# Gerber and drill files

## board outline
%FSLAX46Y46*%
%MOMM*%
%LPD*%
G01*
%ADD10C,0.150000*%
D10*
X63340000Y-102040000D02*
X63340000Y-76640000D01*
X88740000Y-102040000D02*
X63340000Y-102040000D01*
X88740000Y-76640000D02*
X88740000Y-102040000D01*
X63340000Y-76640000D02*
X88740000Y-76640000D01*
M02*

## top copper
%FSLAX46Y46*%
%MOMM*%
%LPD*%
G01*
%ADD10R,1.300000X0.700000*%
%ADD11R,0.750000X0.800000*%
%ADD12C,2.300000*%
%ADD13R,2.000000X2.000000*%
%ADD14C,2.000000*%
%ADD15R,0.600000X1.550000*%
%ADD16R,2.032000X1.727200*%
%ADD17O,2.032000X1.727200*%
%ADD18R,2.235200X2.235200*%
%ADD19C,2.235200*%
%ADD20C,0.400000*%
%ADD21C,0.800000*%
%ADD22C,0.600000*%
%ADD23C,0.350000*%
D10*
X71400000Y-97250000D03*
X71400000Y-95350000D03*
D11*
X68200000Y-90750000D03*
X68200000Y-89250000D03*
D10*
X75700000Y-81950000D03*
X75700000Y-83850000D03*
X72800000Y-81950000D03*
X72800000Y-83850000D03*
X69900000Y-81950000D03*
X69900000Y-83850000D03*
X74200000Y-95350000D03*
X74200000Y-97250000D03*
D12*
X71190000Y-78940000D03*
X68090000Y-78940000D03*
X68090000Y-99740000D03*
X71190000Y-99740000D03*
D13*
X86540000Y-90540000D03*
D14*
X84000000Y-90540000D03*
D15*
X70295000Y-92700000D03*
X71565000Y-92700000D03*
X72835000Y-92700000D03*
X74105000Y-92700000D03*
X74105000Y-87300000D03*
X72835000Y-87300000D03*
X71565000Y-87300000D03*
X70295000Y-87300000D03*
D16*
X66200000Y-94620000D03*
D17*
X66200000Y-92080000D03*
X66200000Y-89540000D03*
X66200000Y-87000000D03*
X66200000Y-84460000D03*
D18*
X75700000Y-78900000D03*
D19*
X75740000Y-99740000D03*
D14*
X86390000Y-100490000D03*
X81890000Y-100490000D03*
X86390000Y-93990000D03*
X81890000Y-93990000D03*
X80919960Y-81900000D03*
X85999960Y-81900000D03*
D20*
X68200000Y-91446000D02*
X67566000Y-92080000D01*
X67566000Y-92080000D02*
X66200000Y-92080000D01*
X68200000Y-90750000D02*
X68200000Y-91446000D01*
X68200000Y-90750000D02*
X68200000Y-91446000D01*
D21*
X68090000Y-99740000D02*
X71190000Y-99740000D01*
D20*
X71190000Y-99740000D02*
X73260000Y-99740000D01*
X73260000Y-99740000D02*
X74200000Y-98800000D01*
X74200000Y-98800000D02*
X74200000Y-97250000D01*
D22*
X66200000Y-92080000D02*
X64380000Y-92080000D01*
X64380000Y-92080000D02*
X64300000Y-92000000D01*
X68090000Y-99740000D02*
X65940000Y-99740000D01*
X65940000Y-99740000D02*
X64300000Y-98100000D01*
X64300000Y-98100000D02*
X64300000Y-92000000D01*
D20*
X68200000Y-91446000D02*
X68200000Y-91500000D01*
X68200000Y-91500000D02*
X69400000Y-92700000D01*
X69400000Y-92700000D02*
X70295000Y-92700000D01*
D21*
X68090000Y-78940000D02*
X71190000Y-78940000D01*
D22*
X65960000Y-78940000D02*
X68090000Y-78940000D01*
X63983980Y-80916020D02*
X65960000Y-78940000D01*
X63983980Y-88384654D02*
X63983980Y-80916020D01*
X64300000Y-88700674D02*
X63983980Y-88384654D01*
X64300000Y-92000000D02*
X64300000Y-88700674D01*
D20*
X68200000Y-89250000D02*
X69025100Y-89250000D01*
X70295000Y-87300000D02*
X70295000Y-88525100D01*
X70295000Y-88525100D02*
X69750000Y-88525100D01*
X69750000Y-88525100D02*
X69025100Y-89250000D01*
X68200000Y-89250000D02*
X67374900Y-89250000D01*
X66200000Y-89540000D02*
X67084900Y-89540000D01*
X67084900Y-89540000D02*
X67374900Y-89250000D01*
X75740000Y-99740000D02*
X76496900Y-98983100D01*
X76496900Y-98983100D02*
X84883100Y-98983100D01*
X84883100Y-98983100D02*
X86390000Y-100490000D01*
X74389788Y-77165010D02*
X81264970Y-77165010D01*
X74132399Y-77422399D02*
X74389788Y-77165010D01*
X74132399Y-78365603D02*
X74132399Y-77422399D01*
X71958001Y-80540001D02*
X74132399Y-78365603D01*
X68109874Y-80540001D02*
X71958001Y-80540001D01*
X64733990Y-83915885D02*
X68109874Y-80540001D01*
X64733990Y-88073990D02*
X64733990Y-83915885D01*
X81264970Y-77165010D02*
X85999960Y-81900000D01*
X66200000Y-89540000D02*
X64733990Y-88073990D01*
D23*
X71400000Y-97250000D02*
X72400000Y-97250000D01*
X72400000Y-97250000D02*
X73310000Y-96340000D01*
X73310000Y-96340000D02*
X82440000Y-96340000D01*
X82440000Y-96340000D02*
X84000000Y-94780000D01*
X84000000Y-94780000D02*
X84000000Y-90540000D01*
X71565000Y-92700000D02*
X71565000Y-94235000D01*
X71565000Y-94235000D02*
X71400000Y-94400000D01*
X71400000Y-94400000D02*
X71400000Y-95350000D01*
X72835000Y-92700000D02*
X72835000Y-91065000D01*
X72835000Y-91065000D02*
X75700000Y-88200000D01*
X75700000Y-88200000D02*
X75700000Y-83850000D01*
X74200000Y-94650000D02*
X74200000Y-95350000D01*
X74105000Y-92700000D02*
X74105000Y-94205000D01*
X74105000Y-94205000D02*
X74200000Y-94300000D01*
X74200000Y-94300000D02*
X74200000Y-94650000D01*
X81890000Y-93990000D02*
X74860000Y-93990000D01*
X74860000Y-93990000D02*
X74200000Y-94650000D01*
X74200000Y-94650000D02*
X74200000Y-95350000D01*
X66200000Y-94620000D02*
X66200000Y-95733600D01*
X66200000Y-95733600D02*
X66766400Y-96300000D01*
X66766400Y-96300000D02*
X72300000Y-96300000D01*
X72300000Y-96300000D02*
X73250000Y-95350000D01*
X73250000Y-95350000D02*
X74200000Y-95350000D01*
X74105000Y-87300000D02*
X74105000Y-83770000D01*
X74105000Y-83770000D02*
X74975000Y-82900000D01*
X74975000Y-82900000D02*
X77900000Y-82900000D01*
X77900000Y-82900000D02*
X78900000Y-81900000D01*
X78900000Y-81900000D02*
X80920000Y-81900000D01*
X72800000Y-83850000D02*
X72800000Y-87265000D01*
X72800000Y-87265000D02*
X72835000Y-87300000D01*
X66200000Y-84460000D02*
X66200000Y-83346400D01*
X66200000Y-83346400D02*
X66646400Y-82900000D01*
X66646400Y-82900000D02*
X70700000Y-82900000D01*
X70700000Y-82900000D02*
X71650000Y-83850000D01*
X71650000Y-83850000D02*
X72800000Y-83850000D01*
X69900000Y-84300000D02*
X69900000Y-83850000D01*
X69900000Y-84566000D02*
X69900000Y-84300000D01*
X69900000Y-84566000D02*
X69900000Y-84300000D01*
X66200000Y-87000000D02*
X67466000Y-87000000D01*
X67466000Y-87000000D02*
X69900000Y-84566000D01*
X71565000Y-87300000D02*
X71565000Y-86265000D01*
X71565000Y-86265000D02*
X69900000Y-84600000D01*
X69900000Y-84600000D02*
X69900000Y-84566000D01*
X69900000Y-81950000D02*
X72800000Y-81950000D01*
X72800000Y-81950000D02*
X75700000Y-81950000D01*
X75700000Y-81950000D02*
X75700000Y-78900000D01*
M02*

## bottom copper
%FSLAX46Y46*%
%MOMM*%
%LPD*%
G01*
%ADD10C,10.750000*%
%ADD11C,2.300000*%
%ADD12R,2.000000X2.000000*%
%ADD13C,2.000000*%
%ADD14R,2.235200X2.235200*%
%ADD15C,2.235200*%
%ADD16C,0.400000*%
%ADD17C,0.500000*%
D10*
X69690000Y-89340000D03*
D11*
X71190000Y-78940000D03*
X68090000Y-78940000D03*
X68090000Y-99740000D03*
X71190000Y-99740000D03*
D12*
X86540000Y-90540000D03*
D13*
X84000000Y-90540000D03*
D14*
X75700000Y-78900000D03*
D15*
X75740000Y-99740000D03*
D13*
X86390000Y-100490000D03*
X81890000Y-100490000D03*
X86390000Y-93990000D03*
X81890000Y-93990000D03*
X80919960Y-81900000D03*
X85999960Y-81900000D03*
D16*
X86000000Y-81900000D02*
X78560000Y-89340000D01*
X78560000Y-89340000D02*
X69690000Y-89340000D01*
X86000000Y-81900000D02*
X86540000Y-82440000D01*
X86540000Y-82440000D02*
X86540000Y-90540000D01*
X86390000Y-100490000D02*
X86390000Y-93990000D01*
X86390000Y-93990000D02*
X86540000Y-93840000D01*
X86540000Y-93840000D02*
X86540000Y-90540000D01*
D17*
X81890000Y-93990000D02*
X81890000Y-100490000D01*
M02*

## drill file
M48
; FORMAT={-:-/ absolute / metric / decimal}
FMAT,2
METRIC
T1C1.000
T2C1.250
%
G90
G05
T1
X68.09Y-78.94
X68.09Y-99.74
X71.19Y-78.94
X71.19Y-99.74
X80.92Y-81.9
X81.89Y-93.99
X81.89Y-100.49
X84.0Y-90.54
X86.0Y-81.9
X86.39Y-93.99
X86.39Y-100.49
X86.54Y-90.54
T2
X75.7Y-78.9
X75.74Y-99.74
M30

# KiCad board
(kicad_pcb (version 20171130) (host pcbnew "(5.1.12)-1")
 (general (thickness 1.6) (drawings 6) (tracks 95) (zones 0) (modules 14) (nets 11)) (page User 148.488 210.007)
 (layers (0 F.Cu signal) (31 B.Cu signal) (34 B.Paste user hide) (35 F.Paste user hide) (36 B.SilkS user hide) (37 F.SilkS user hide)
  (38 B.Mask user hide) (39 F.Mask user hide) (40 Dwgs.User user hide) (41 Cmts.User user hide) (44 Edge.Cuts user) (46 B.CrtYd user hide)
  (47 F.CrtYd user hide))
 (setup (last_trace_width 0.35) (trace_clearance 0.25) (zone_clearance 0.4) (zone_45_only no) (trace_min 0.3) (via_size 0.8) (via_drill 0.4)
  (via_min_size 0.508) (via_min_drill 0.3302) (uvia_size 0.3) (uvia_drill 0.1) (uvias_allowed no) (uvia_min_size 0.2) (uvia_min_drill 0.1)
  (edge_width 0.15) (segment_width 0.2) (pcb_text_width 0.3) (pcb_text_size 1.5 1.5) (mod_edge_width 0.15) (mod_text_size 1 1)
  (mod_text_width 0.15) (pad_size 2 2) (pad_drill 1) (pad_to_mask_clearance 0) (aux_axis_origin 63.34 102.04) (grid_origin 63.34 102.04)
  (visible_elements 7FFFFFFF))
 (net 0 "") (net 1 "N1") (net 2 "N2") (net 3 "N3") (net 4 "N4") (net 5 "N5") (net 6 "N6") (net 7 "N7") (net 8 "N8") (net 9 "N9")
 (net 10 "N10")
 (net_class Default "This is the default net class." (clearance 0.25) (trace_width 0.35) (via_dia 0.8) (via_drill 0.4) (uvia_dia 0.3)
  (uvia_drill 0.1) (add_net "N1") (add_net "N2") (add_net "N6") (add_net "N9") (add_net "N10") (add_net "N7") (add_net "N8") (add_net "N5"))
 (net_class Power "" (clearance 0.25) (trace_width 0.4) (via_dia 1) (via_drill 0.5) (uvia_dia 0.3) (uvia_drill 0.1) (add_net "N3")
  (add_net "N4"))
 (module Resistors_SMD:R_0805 (layer F.Cu) (at 71.4 96.3 90)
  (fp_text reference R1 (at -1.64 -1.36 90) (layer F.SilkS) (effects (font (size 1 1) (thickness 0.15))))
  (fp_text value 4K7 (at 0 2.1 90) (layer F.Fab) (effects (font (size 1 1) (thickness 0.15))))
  (pad 1 smd rect (at -0.95 0 90) (size 0.7 1.3) (layers F.Cu F.Paste F.Mask) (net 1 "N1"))
  (pad 2 smd rect (at 0.95 0 90) (size 0.7 1.3) (layers F.Cu F.Paste F.Mask) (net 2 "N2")))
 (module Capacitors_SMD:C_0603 (layer F.Cu) (at 68.2 90 90)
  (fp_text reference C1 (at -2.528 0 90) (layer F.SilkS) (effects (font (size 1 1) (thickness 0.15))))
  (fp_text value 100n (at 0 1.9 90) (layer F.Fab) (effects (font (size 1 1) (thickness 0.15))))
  (pad 1 smd rect (at -0.75 0 90) (size 0.8 0.75) (layers F.Cu F.Paste F.Mask) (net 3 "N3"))
  (pad 2 smd rect (at 0.75 0 90) (size 0.8 0.75) (layers F.Cu F.Paste F.Mask) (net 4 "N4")))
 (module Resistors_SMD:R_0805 (layer F.Cu) (at 75.7 82.9 270)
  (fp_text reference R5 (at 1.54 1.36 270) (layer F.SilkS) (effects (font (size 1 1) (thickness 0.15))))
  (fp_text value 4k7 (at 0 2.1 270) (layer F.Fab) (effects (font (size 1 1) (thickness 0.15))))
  (pad 1 smd rect (at -0.95 0 270) (size 0.7 1.3) (layers F.Cu F.Paste F.Mask) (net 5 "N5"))
  (pad 2 smd rect (at 0.95 0 270) (size 0.7 1.3) (layers F.Cu F.Paste F.Mask) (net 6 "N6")))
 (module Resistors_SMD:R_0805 (layer F.Cu) (at 72.8 82.9 270)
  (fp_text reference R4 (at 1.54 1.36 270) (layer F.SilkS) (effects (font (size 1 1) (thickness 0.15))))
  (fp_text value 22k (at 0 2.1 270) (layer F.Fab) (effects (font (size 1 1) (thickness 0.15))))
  (pad 1 smd rect (at -0.95 0 270) (size 0.7 1.3) (layers F.Cu F.Paste F.Mask) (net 5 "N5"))
  (pad 2 smd rect (at 0.95 0 270) (size 0.7 1.3) (layers F.Cu F.Paste F.Mask) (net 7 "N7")))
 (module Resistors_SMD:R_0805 (layer F.Cu) (at 69.9 82.9 270)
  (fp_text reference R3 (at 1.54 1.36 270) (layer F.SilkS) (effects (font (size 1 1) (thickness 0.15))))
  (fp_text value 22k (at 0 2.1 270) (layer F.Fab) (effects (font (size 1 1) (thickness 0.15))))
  (pad 1 smd rect (at -0.95 0 270) (size 0.7 1.3) (layers F.Cu F.Paste F.Mask) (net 5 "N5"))
  (pad 2 smd rect (at 0.95 0 270) (size 0.7 1.3) (layers F.Cu F.Paste F.Mask) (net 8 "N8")))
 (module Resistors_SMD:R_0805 (layer F.Cu) (at 74.2 96.3 270)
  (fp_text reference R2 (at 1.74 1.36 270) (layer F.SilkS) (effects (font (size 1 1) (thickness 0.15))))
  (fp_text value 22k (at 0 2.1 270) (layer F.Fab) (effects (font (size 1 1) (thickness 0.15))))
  (pad 1 smd rect (at -0.95 0 270) (size 0.7 1.3) (layers F.Cu F.Paste F.Mask) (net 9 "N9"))
  (pad 2 smd rect (at 0.95 0 270) (size 0.7 1.3) (layers F.Cu F.Paste F.Mask) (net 3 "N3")))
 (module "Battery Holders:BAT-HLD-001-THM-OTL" (layer B.Cu) (at 69.69 89.34 90)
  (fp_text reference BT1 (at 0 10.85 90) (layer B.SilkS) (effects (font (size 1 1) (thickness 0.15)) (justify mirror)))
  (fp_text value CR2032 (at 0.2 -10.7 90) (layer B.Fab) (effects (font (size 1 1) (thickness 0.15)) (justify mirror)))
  (pad 2 smd circle (at 0 0 90) (size 10.75 10.75) (layers B.Cu B.Mask) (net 4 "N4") (solder_mask_margin 4) (clearance 2.5) (zone_connect 1)
   (thermal_gap 4))
  (pad 1 thru_hole circle (at 10.4 1.5 90) (size 2.3 2.3) (drill 1) (layers *.Cu *.Mask B.SilkS) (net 3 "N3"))
  (pad 1 thru_hole circle (at 10.4 -1.6 90) (size 2.3 2.3) (drill 1) (layers *.Cu *.Mask B.SilkS) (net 3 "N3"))
  (pad 1 thru_hole circle (at -10.4 -1.6 90) (size 2.3 2.3) (drill 1) (layers *.Cu *.Mask B.SilkS) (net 3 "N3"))
  (pad 1 thru_hole circle (at -10.4 1.5 90) (size 2.3 2.3) (drill 1) (layers *.Cu *.Mask B.SilkS) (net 3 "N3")))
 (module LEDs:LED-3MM (layer F.Cu) (at 86.54 90.54 180)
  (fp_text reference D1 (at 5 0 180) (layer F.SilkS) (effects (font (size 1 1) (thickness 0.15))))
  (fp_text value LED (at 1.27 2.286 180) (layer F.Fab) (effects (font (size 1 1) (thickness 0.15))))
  (pad 1 thru_hole rect (at 0 0 270) (size 2 2) (drill 1) (layers *.Cu *.Mask F.SilkS) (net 4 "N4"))
  (pad 2 thru_hole circle (at 2.54 0 180) (size 2 2) (drill 1) (layers *.Cu *.Mask F.SilkS) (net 1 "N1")))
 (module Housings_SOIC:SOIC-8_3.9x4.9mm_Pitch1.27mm (layer F.Cu) (at 72.2 90 90)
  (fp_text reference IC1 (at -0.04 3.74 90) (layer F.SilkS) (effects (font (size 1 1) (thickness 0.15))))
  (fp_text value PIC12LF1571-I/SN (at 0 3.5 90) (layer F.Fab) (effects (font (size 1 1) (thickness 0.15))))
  (pad 1 smd rect (at -2.7 -1.905 90) (size 1.55 0.6) (layers F.Cu F.Paste F.Mask) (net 3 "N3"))
  (pad 2 smd rect (at -2.7 -0.635 90) (size 1.55 0.6) (layers F.Cu F.Paste F.Mask) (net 2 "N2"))
  (pad 3 smd rect (at -2.7 0.635 90) (size 1.55 0.6) (layers F.Cu F.Paste F.Mask) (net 6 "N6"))
  (pad 4 smd rect (at -2.7 1.905 90) (size 1.55 0.6) (layers F.Cu F.Paste F.Mask) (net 9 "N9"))
  (pad 5 smd rect (at 2.7 1.905 90) (size 1.55 0.6) (layers F.Cu F.Paste F.Mask) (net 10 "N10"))
  (pad 6 smd rect (at 2.7 0.635 90) (size 1.55 0.6) (layers F.Cu F.Paste F.Mask) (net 7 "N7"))
  (pad 7 smd rect (at 2.7 -0.635 90) (size 1.55 0.6) (layers F.Cu F.Paste F.Mask) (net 8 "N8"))
  (pad 8 smd rect (at 2.7 -1.905 90) (size 1.55 0.6) (layers F.Cu F.Paste F.Mask) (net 4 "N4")))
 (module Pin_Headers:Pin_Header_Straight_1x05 (layer F.Cu) (at 66.2 94.62 180)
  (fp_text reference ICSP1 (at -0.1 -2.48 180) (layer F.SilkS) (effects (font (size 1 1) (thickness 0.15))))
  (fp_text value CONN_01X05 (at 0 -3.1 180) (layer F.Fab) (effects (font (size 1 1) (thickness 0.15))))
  (pad 1 smd rect (at 0 0 180) (size 2.032 1.7272) (layers F.Cu F.Mask) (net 9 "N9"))
  (pad 2 smd oval (at 0 2.54 180) (size 2.032 1.7272) (layers F.Cu F.Mask) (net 3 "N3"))
  (pad 3 smd oval (at 0 5.08 180) (size 2.032 1.7272) (layers F.Cu F.Mask) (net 4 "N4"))
  (pad 4 smd oval (at 0 7.62 180) (size 2.032 1.7272) (layers F.Cu F.Mask) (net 8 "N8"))
  (pad 5 smd oval (at 0 10.16 180) (size 2.032 1.7272) (layers F.Cu F.Mask) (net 7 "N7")))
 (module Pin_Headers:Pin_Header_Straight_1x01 (layer F.Cu) (at 75.7 78.9)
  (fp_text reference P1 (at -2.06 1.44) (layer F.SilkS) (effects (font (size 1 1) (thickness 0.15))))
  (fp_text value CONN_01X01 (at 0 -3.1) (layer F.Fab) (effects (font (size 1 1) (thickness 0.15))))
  (pad 1 thru_hole rect (at 0 0) (size 2.2352 2.2352) (drill 1.25) (layers *.Cu *.Mask F.SilkS) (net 5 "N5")))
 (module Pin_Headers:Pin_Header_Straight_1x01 (layer F.Cu) (at 75.74 99.74)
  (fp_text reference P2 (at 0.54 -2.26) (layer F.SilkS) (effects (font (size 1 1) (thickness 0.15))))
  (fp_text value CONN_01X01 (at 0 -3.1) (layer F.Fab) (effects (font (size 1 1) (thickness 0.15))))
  (pad 1 thru_hole circle (at 0 0) (size 2.2352 2.2352) (drill 1.25) (layers *.Cu *.Mask F.SilkS) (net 4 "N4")))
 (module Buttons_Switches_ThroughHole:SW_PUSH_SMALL (layer F.Cu) (at 84.14 97.24 270)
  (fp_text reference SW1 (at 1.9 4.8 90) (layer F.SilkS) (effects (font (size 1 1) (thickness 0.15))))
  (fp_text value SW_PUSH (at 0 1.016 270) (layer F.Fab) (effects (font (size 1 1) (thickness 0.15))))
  (pad 1 thru_hole circle (at 3.25 -2.25 270) (size 2 2) (drill 1) (layers *.Cu *.Mask F.SilkS) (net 4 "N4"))
  (pad 2 thru_hole circle (at 3.25 2.25 270) (size 2 2) (drill 1) (layers *.Cu *.Mask F.SilkS) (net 9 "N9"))
  (pad 1 thru_hole circle (at -3.25 -2.25 270) (size 2 2) (drill 1) (layers *.Cu *.Mask F.SilkS) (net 4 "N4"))
  (pad 2 thru_hole circle (at -3.25 2.25 270) (size 2 2) (drill 1) (layers *.Cu *.Mask F.SilkS) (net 9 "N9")))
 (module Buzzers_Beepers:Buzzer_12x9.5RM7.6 (layer F.Cu) (at 83.4498 81.9)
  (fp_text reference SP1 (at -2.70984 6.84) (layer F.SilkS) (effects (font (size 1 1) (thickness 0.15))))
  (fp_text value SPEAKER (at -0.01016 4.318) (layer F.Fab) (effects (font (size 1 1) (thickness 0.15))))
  (pad 1 thru_hole circle (at -2.52984 0) (size 2 2) (drill 1) (layers *.Cu *.Mask F.SilkS) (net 10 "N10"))
  (pad 2 thru_hole circle (at 2.55016 0) (size 2 2) (drill 1) (layers *.Cu *.Mask F.SilkS) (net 4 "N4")))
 (gr_line (start 63.34 102.04) (end 63.34 76.64) (layer Edge.Cuts) (width 0.15))
 (gr_line (start 88.74 102.04) (end 63.34 102.04) (layer Edge.Cuts) (width 0.15))
 (gr_line (start 88.74 76.64) (end 88.74 102.04) (layer Edge.Cuts) (width 0.15))
 (gr_line (start 63.34 76.64) (end 88.74 76.64) (layer Edge.Cuts) (width 0.15))
 (segment (start 68.2 91.446) (end 67.566 92.08) (width 0.4) (layer F.Cu) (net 3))
 (segment (start 67.566 92.08) (end 66.2 92.08) (width 0.4) (layer F.Cu) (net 3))
 (segment (start 68.2 90.75) (end 68.2 91.446) (width 0.4) (layer F.Cu) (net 3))
 (segment (start 68.2 90.75) (end 68.2 91.446) (width 0.4) (layer F.Cu) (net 3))
 (segment (start 68.09 99.74) (end 71.19 99.74) (width 0.8) (layer F.Cu) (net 3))
 (segment (start 71.19 99.74) (end 73.26 99.74) (width 0.4) (layer F.Cu) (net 3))
 (segment (start 73.26 99.74) (end 74.2 98.8) (width 0.4) (layer F.Cu) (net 3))
 (segment (start 74.2 98.8) (end 74.2 97.25) (width 0.4) (layer F.Cu) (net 3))
 (segment (start 66.2 92.08) (end 64.38 92.08) (width 0.6) (layer F.Cu) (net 3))
 (segment (start 64.38 92.08) (end 64.3 92) (width 0.6) (layer F.Cu) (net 3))
 (segment (start 68.09 99.74) (end 65.94 99.74) (width 0.6) (layer F.Cu) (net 3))
 (segment (start 65.94 99.74) (end 64.3 98.1) (width 0.6) (layer F.Cu) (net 3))
 (segment (start 64.3 98.1) (end 64.3 92) (width 0.6) (layer F.Cu) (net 3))
 (segment (start 68.2 91.446) (end 68.2 91.5) (width 0.4) (layer F.Cu) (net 3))
 (segment (start 68.2 91.5) (end 69.4 92.7) (width 0.4) (layer F.Cu) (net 3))
 (segment (start 69.4 92.7) (end 70.295 92.7) (width 0.4) (layer F.Cu) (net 3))
 (segment (start 68.09 78.94) (end 71.19 78.94) (width 0.8) (layer F.Cu) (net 3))
 (segment (start 65.96 78.94) (end 68.09 78.94) (width 0.6) (layer F.Cu) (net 3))
 (segment (start 63.98398 80.91602) (end 65.96 78.94) (width 0.6) (layer F.Cu) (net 3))
 (segment (start 63.98398 88.384654) (end 63.98398 80.91602) (width 0.6) (layer F.Cu) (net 3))
 (segment (start 64.3 88.700674) (end 63.98398 88.384654) (width 0.6) (layer F.Cu) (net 3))
 (segment (start 64.3 92) (end 64.3 88.700674) (width 0.6) (layer F.Cu) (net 3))
 (segment (start 86 81.9) (end 78.56 89.34) (width 0.4) (layer B.Cu) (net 4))
 (segment (start 78.56 89.34) (end 69.69 89.34) (width 0.4) (layer B.Cu) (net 4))
 (segment (start 86 81.9) (end 86.54 82.44) (width 0.4) (layer B.Cu) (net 4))
 (segment (start 86.54 82.44) (end 86.54 90.54) (width 0.4) (layer B.Cu) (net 4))
 (segment (start 68.2 89.25) (end 69.0251 89.25) (width 0.4) (layer F.Cu) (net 4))
 (segment (start 70.295 87.3) (end 70.295 88.5251) (width 0.4) (layer F.Cu) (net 4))
 (segment (start 70.295 88.5251) (end 69.75 88.5251) (width 0.4) (layer F.Cu) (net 4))
 (segment (start 69.75 88.5251) (end 69.0251 89.25) (width 0.4) (layer F.Cu) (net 4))
 (segment (start 68.2 89.25) (end 67.3749 89.25) (width 0.4) (layer F.Cu) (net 4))
 (segment (start 66.2 89.54) (end 67.0849 89.54) (width 0.4) (layer F.Cu) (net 4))
 (segment (start 67.0849 89.54) (end 67.3749 89.25) (width 0.4) (layer F.Cu) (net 4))
 (segment (start 75.74 99.74) (end 76.4969 98.9831) (width 0.4) (layer F.Cu) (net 4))
 (segment (start 76.4969 98.9831) (end 84.8831 98.9831) (width 0.4) (layer F.Cu) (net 4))
 (segment (start 84.8831 98.9831) (end 86.39 100.49) (width 0.4) (layer F.Cu) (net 4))
 (segment (start 86.39 100.49) (end 86.39 93.99) (width 0.4) (layer B.Cu) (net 4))
 (segment (start 86.39 93.99) (end 86.54 93.84) (width 0.4) (layer B.Cu) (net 4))
 (segment (start 86.54 93.84) (end 86.54 90.54) (width 0.4) (layer B.Cu) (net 4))
 (segment (start 74.389788 77.16501) (end 81.26497 77.16501) (width 0.4) (layer F.Cu) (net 4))
 (segment (start 74.132399 77.422399) (end 74.389788 77.16501) (width 0.4) (layer F.Cu) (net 4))
 (segment (start 74.132399 78.365603) (end 74.132399 77.422399) (width 0.4) (layer F.Cu) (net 4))
 (segment (start 71.958001 80.540001) (end 74.132399 78.365603) (width 0.4) (layer F.Cu) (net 4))
 (segment (start 68.109874 80.540001) (end 71.958001 80.540001) (width 0.4) (layer F.Cu) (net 4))
 (segment (start 64.73399 83.915885) (end 68.109874 80.540001) (width 0.4) (layer F.Cu) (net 4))
 (segment (start 64.73399 88.07399) (end 64.73399 83.915885) (width 0.4) (layer F.Cu) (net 4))
 (segment (start 81.26497 77.16501) (end 85.99996 81.9) (width 0.4) (layer F.Cu) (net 4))
 (segment (start 66.2 89.54) (end 64.73399 88.07399) (width 0.4) (layer F.Cu) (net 4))
 (segment (start 71.4 97.25) (end 72.4 97.25) (width 0.35) (layer F.Cu) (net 1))
 (segment (start 72.4 97.25) (end 73.31 96.34) (width 0.35) (layer F.Cu) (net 1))
 (segment (start 73.31 96.34) (end 82.44 96.34) (width 0.35) (layer F.Cu) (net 1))
 (segment (start 82.44 96.34) (end 84 94.78) (width 0.35) (layer F.Cu) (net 1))
 (segment (start 84 94.78) (end 84 90.54) (width 0.35) (layer F.Cu) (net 1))
 (segment (start 71.565 92.7) (end 71.565 94.235) (width 0.35) (layer F.Cu) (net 2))
 (segment (start 71.565 94.235) (end 71.4 94.4) (width 0.35) (layer F.Cu) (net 2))
 (segment (start 71.4 94.4) (end 71.4 95.35) (width 0.35) (layer F.Cu) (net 2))
 (segment (start 72.835 92.7) (end 72.835 91.065) (width 0.35) (layer F.Cu) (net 6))
 (segment (start 72.835 91.065) (end 75.7 88.2) (width 0.35) (layer F.Cu) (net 6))
 (segment (start 75.7 88.2) (end 75.7 83.85) (width 0.35) (layer F.Cu) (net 6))
 (segment (start 74.2 94.65) (end 74.2 95.35) (width 0.35) (layer F.Cu) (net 9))
 (segment (start 74.105 92.7) (end 74.105 94.205) (width 0.35) (layer F.Cu) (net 9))
 (segment (start 74.105 94.205) (end 74.2 94.3) (width 0.35) (layer F.Cu) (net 9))
 (segment (start 74.2 94.3) (end 74.2 94.65) (width 0.35) (layer F.Cu) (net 9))
 (segment (start 81.89 93.99) (end 74.86 93.99) (width 0.35) (layer F.Cu) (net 9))
 (segment (start 74.86 93.99) (end 74.2 94.65) (width 0.35) (layer F.Cu) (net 9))
 (segment (start 81.89 93.99) (end 81.89 100.49) (width 0.5) (layer B.Cu) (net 9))
 (segment (start 74.2 94.65) (end 74.2 95.35) (width 0.35) (layer F.Cu) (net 9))
 (segment (start 66.2 94.62) (end 66.2 95.7336) (width 0.35) (layer F.Cu) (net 9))
 (segment (start 66.2 95.7336) (end 66.7664 96.3) (width 0.35) (layer F.Cu) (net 9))
 (segment (start 66.7664 96.3) (end 72.3 96.3) (width 0.35) (layer F.Cu) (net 9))
 (segment (start 72.3 96.3) (end 73.25 95.35) (width 0.35) (layer F.Cu) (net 9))
 (segment (start 73.25 95.35) (end 74.2 95.35) (width 0.35) (layer F.Cu) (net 9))
 (segment (start 74.105 87.3) (end 74.105 83.77) (width 0.35) (layer F.Cu) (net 10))
 (segment (start 74.105 83.77) (end 74.975 82.9) (width 0.35) (layer F.Cu) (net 10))
 (segment (start 74.975 82.9) (end 77.9 82.9) (width 0.35) (layer F.Cu) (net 10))
 (segment (start 77.9 82.9) (end 78.9 81.9) (width 0.35) (layer F.Cu) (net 10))
 (segment (start 78.9 81.9) (end 80.92 81.9) (width 0.35) (layer F.Cu) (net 10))
 (segment (start 72.8 83.85) (end 72.8 87.265) (width 0.35) (layer F.Cu) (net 7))
 (segment (start 72.8 87.265) (end 72.835 87.3) (width 0.35) (layer F.Cu) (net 7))
 (segment (start 66.2 84.46) (end 66.2 83.3464) (width 0.35) (layer F.Cu) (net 7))
 (segment (start 66.2 83.3464) (end 66.6464 82.9) (width 0.35) (layer F.Cu) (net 7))
 (segment (start 66.6464 82.9) (end 70.7 82.9) (width 0.35) (layer F.Cu) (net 7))
 (segment (start 70.7 82.9) (end 71.65 83.85) (width 0.35) (layer F.Cu) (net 7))
 (segment (start 71.65 83.85) (end 72.8 83.85) (width 0.35) (layer F.Cu) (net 7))
 (segment (start 69.9 84.3) (end 69.9 83.85) (width 0.35) (layer F.Cu) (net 8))
 (segment (start 69.9 84.566) (end 69.9 84.3) (width 0.35) (layer F.Cu) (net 8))
 (segment (start 69.9 84.566) (end 69.9 84.3) (width 0.35) (layer F.Cu) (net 8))
 (segment (start 66.2 87) (end 67.466 87) (width 0.35) (layer F.Cu) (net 8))
 (segment (start 67.466 87) (end 69.9 84.566) (width 0.35) (layer F.Cu) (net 8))
 (segment (start 71.565 87.3) (end 71.565 86.265) (width 0.35) (layer F.Cu) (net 8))
 (segment (start 71.565 86.265) (end 69.9 84.6) (width 0.35) (layer F.Cu) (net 8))
 (segment (start 69.9 84.6) (end 69.9 84.566) (width 0.35) (layer F.Cu) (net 8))
 (segment (start 69.9 81.95) (end 72.8 81.95) (width 0.35) (layer F.Cu) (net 5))
 (segment (start 72.8 81.95) (end 75.7 81.95) (width 0.35) (layer F.Cu) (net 5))
 (segment (start 75.7 81.95) (end 75.7 78.9) (width 0.35) (layer F.Cu) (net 5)))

